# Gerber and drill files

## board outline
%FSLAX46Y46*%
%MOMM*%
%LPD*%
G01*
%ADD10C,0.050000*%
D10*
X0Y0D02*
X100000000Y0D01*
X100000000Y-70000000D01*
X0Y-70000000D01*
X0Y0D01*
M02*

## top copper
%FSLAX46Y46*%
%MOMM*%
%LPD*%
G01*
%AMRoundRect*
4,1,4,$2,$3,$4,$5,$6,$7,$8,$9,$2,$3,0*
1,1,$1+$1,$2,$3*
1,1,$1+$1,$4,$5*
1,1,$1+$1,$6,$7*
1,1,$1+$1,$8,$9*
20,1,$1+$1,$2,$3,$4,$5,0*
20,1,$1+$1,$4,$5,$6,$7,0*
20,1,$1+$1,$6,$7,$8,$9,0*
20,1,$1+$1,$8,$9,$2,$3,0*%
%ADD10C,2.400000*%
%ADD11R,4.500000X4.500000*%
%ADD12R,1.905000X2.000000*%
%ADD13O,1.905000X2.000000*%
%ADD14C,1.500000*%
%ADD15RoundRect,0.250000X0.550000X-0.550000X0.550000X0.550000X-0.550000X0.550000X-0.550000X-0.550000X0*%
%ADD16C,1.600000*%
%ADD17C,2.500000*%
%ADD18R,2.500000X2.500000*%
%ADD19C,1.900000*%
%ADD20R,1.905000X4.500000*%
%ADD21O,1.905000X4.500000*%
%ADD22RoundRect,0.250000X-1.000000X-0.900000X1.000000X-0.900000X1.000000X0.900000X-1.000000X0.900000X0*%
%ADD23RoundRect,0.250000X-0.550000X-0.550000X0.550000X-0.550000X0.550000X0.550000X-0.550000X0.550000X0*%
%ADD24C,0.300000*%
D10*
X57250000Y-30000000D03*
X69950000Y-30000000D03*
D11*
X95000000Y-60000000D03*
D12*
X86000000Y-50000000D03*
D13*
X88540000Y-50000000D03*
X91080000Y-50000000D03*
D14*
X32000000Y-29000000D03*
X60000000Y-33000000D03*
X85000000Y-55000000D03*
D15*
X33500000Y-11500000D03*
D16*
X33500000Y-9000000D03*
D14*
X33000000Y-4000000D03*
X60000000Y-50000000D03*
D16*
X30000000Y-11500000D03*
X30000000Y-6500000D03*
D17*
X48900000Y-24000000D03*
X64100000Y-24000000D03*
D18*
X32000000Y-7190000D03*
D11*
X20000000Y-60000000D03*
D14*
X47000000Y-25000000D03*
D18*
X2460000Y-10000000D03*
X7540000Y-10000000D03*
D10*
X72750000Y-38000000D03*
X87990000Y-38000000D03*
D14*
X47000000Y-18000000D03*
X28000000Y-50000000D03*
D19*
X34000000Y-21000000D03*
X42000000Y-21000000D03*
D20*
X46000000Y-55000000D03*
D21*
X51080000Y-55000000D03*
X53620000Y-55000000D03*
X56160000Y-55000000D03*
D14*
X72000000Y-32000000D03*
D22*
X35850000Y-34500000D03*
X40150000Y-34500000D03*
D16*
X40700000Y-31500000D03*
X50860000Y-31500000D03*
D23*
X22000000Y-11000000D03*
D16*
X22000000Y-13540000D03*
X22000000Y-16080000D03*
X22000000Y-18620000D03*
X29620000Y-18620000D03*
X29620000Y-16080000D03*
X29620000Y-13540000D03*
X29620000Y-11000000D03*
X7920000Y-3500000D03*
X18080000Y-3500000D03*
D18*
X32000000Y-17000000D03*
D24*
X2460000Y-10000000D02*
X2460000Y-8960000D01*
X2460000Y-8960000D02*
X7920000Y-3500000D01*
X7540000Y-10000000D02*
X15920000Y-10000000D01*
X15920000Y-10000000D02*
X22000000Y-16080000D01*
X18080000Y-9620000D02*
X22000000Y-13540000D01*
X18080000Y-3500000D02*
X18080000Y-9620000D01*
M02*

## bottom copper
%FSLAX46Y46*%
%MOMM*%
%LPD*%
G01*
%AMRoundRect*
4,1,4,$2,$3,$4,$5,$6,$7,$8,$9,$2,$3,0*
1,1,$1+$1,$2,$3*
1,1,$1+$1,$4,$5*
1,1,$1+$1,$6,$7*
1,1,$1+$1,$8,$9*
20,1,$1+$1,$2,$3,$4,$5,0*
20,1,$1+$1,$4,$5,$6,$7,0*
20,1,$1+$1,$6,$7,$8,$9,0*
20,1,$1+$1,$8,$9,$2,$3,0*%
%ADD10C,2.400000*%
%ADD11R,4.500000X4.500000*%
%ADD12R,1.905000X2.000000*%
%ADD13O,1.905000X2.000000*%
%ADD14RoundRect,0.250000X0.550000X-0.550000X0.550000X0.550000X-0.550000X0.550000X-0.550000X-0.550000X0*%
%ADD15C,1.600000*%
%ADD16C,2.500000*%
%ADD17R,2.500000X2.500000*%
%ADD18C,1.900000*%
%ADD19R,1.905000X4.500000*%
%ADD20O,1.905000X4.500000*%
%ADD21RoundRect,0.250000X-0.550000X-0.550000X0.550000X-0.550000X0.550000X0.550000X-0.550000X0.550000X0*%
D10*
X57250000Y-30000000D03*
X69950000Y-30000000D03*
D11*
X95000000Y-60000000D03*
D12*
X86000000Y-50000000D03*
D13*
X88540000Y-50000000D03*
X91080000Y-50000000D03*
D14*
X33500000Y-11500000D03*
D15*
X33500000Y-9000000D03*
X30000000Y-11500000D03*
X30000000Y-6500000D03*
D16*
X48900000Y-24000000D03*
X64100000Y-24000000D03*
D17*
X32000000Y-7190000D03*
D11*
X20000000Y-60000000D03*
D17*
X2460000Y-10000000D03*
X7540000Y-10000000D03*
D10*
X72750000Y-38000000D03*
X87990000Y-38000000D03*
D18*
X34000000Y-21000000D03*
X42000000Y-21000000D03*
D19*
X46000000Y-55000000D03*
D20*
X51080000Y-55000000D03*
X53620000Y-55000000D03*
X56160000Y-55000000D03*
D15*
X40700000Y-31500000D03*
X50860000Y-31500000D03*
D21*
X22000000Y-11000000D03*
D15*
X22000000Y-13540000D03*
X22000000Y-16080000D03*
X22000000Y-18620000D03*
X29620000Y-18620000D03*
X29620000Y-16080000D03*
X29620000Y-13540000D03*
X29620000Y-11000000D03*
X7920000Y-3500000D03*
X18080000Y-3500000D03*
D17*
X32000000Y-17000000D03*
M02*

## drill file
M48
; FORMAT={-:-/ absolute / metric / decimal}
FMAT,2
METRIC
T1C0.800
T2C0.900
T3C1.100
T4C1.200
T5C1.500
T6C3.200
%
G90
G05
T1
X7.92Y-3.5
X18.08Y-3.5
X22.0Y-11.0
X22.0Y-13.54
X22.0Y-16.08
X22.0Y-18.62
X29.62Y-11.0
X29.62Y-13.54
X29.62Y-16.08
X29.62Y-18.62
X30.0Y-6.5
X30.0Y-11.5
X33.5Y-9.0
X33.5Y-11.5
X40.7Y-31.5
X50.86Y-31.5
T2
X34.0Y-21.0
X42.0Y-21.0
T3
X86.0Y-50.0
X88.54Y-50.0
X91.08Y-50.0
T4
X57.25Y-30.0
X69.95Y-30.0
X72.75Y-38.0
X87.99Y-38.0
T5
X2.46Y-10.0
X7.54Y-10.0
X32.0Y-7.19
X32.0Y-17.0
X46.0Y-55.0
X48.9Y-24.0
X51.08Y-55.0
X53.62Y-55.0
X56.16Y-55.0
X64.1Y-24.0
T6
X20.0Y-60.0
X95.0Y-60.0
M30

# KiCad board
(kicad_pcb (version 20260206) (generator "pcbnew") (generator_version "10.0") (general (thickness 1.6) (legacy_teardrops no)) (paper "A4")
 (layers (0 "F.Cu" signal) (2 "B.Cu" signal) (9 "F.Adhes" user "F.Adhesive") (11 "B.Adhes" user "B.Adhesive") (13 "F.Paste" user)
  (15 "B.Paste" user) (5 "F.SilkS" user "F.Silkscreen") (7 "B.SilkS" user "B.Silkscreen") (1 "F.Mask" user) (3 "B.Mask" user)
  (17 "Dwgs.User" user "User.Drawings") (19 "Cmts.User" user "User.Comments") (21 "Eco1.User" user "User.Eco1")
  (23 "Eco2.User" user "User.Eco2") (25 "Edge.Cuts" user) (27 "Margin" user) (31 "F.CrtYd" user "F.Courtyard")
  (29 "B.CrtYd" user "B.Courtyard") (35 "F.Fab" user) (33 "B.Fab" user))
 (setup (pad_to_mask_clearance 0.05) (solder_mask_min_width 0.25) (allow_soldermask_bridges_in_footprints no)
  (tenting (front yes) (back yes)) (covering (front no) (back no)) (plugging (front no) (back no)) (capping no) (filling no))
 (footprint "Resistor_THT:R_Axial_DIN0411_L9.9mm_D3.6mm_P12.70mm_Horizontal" (layer "F.Cu") (at 57.25 30)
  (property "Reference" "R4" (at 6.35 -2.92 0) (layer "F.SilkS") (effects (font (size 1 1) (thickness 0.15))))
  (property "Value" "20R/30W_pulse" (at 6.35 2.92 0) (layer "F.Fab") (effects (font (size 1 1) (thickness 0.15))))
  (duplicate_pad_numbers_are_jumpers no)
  (pad "1" thru_hole circle (at 0 0) (size 2.4 2.4) (drill 1.2) (layers "*.Cu" "*.Mask") (remove_unused_layers no) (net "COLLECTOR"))
  (pad "2" thru_hole circle (at 12.7 0) (size 2.4 2.4) (drill 1.2) (layers "*.Cu" "*.Mask") (remove_unused_layers no)
   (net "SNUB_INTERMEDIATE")))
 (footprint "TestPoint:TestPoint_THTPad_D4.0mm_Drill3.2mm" (layer "F.Cu") (at 95 60)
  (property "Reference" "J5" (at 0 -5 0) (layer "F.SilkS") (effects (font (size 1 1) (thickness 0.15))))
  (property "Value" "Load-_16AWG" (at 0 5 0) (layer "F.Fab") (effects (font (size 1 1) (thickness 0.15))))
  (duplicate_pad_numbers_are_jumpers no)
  (pad "1" thru_hole rect (at 0 0) (size 4.5 4.5) (drill 3.2) (layers "*.Cu" "*.Mask") (remove_unused_layers no) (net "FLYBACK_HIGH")))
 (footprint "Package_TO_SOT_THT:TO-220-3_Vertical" (layer "F.Cu") (at 86 50)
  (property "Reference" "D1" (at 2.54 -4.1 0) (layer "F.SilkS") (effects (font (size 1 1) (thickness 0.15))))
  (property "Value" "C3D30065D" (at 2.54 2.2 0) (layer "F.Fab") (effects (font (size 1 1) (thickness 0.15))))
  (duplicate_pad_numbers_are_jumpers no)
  (pad "1" thru_hole rect (at 0 0) (size 1.905 2) (drill 1.1) (layers "*.Cu" "*.Mask") (remove_unused_layers no) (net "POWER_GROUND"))
  (pad "2" thru_hole oval (at 2.54 0) (size 1.905 2) (drill 1.1) (layers "*.Cu" "*.Mask") (remove_unused_layers no) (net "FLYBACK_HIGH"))
  (pad "3" thru_hole oval (at 5.08 0) (size 1.905 2) (drill 1.1) (layers "*.Cu" "*.Mask") (remove_unused_layers no) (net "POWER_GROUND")))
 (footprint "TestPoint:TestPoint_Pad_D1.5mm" (layer "F.Cu") (at 32 29)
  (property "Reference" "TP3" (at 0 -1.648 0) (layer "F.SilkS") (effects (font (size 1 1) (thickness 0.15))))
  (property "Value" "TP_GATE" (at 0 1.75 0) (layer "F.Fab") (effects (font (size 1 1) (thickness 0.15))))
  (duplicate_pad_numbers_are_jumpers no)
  (pad "1" smd circle (at 0 0) (size 1.5 1.5) (layers "F.Cu" "F.Mask") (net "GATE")))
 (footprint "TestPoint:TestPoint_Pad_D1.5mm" (layer "F.Cu") (at 60 33)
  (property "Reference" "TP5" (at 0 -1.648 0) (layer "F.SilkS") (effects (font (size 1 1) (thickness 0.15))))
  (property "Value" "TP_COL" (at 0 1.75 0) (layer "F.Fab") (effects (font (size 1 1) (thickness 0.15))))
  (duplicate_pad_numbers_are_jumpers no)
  (pad "1" smd circle (at 0 0) (size 1.5 1.5) (layers "F.Cu" "F.Mask") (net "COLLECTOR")))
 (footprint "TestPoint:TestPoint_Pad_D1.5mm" (layer "F.Cu") (at 85 55)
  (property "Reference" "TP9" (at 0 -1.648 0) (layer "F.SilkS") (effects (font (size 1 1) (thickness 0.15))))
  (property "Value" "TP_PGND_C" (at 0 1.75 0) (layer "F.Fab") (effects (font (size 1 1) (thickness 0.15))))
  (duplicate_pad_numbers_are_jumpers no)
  (pad "1" smd circle (at 0 0) (size 1.5 1.5) (layers "F.Cu" "F.Mask") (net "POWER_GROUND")))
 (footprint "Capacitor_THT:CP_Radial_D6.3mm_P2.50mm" (layer "F.Cu") (at 33.5 11.5 90)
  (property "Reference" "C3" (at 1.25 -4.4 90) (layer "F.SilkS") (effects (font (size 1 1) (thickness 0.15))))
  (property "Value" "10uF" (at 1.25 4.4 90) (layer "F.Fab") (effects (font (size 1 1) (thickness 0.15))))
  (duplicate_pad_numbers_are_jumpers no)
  (pad "1" thru_hole roundrect (at 0 0 90) (size 1.6 1.6) (drill 0.8) (layers "*.Cu" "*.Mask") (remove_unused_layers no)
   (roundrect_rratio 0.15625) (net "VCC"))
  (pad "2" thru_hole circle (at 2.5 0 90) (size 1.6 1.6) (drill 0.8) (layers "*.Cu" "*.Mask") (remove_unused_layers no)
   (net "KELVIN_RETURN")))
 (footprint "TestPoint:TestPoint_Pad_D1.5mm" (layer "F.Cu") (at 33 4)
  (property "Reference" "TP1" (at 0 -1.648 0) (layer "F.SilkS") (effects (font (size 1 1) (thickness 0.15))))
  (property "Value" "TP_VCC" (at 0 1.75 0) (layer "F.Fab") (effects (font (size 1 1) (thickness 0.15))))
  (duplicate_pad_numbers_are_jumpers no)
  (pad "1" smd circle (at 0 0) (size 1.5 1.5) (layers "F.Cu" "F.Mask") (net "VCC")))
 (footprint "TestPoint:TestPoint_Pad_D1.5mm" (layer "F.Cu") (at 60 50)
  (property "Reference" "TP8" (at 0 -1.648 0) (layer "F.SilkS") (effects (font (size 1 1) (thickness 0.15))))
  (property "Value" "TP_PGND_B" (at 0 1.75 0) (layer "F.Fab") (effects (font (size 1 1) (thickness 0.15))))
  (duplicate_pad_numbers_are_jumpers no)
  (pad "1" smd circle (at 0 0) (size 1.5 1.5) (layers "F.Cu" "F.Mask") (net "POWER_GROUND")))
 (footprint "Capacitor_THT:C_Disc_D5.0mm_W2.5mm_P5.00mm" (layer "F.Cu") (at 30 11.5 90)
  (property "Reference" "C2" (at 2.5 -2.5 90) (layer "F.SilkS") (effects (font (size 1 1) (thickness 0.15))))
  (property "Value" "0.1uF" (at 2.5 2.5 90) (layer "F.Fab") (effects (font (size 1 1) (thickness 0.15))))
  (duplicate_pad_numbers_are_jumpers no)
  (pad "1" thru_hole circle (at 0 0 90) (size 1.6 1.6) (drill 0.8) (layers "*.Cu" "*.Mask") (remove_unused_layers no) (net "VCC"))
  (pad "2" thru_hole circle (at 5 0 90) (size 1.6 1.6) (drill 0.8) (layers "*.Cu" "*.Mask") (remove_unused_layers no) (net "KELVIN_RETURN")))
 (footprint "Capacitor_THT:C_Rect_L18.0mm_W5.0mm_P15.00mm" (layer "F.Cu") (at 56.5 24)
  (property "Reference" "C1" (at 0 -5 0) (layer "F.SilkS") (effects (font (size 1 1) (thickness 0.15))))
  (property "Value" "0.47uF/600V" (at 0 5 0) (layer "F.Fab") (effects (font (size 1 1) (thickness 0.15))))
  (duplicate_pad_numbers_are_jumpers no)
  (pad "1" thru_hole circle (at -7.6 0) (size 2.5 2.5) (drill 1.5) (layers "*.Cu" "*.Mask") (remove_unused_layers no) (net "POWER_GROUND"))
  (pad "2" thru_hole circle (at 7.6 0) (size 2.5 2.5) (drill 1.5) (layers "*.Cu" "*.Mask") (remove_unused_layers no)
   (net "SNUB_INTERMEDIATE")))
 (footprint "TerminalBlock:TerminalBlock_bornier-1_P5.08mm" (layer "F.Cu") (at 32 7.19)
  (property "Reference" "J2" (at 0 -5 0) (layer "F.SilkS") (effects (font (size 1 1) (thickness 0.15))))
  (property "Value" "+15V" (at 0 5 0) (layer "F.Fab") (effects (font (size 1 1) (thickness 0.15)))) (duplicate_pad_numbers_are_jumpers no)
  (pad "1" thru_hole rect (at 0 0) (size 2.5 2.5) (drill 1.5) (layers "*.Cu" "*.Mask") (remove_unused_layers no) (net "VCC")))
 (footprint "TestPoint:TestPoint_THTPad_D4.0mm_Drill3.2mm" (layer "F.Cu") (at 20 60)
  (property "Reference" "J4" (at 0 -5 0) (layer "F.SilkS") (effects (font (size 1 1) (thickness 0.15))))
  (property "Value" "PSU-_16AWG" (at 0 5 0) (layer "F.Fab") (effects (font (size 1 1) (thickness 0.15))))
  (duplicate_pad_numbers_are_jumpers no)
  (pad "1" thru_hole rect (at 0 0) (size 4.5 4.5) (drill 3.2) (layers "*.Cu" "*.Mask") (remove_unused_layers no) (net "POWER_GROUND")))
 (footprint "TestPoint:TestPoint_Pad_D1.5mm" (layer "F.Cu") (at 47 25)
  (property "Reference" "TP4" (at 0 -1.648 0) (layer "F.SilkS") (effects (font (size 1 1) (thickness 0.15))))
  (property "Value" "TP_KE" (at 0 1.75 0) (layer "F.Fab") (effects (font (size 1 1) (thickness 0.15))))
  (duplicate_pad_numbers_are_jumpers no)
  (pad "1" smd circle (at 0 0) (size 1.5 1.5) (layers "F.Cu" "F.Mask") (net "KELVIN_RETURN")))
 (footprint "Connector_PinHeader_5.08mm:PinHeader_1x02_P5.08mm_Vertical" (layer "F.Cu") (at 5 10 90)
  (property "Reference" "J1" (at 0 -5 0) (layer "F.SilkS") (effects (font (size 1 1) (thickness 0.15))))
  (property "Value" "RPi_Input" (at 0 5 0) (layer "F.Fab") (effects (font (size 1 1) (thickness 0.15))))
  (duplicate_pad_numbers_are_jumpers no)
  (pad "1" thru_hole rect (at 0 -2.54) (size 2.5 2.5) (drill 1.5) (layers "*.Cu" "*.Mask") (remove_unused_layers no) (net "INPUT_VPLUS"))
  (pad "2" thru_hole rect (at 0 2.54) (size 2.5 2.5) (drill 1.5) (layers "*.Cu" "*.Mask") (remove_unused_layers no) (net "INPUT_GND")))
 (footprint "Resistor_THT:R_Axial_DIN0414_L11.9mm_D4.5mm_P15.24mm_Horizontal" (layer "F.Cu") (at 72.75 38)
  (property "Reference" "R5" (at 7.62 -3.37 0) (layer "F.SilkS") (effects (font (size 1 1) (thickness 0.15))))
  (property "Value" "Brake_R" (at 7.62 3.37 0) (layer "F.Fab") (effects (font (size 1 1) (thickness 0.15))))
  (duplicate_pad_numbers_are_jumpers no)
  (pad "1" thru_hole circle (at 0 0) (size 2.4 2.4) (drill 1.2) (layers "*.Cu" "*.Mask") (remove_unused_layers no) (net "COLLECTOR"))
  (pad "2" thru_hole circle (at 15.24 0) (size 2.4 2.4) (drill 1.2) (layers "*.Cu" "*.Mask") (remove_unused_layers no) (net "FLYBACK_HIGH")))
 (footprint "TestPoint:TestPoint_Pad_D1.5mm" (layer "F.Cu") (at 47 18)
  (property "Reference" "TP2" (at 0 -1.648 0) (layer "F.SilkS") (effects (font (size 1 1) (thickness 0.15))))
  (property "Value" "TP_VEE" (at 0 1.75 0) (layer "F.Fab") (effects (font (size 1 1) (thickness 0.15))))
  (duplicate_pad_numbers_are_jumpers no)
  (pad "1" smd circle (at 0 0) (size 1.5 1.5) (layers "F.Cu" "F.Mask") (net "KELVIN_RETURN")))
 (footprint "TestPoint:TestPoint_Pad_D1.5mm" (layer "F.Cu") (at 28 50)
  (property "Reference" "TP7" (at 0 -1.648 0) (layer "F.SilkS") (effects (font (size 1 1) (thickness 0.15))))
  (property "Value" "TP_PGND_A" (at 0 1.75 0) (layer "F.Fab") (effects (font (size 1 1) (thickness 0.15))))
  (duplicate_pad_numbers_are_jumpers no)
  (pad "1" smd circle (at 0 0) (size 1.5 1.5) (layers "F.Cu" "F.Mask") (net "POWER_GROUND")))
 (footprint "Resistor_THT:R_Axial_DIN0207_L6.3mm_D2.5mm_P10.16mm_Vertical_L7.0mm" (layer "F.Cu") (at 38 21 90)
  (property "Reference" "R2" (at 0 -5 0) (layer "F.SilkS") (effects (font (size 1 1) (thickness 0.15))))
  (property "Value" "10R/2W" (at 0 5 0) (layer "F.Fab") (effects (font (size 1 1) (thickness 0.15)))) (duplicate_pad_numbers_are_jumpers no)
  (pad "1" thru_hole circle (at 0 -4) (size 1.9 1.9) (drill 0.9) (layers "*.Cu" "*.Mask") (remove_unused_layers no) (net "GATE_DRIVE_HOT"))
  (pad "2" thru_hole circle (at 0 4) (size 1.9 1.9) (drill 0.9) (layers "*.Cu" "*.Mask") (remove_unused_layers no) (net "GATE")))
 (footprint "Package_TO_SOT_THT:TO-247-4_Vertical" (layer "F.Cu") (at 46 55)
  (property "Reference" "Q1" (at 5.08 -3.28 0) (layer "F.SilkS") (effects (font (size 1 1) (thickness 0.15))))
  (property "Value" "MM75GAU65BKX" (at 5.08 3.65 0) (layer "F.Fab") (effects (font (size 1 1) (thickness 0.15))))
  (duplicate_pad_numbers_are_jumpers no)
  (pad "1" thru_hole rect (at 0 0) (size 1.905 4.5) (drill 1.5) (layers "*.Cu" "*.Mask") (remove_unused_layers no) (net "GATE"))
  (pad "2" thru_hole oval (at 5.08 0) (size 1.905 4.5) (drill 1.5) (layers "*.Cu" "*.Mask") (remove_unused_layers no) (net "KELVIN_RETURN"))
  (pad "3" thru_hole oval (at 7.62 0) (size 1.905 4.5) (drill 1.5) (layers "*.Cu" "*.Mask") (remove_unused_layers no) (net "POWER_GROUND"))
  (pad "4" thru_hole oval (at 10.16 0) (size 1.905 4.5) (drill 1.5) (layers "*.Cu" "*.Mask") (remove_unused_layers no) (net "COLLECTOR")))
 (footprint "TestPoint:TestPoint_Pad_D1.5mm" (layer "F.Cu") (at 72 32)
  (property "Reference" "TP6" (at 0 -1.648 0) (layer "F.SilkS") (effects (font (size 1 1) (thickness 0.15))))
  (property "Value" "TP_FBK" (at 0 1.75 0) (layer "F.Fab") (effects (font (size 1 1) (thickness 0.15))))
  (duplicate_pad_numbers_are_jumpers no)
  (pad "1" smd circle (at 0 0) (size 1.5 1.5) (layers "F.Cu" "F.Mask") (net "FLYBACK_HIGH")))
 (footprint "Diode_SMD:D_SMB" (layer "F.Cu") (at 38 34.5)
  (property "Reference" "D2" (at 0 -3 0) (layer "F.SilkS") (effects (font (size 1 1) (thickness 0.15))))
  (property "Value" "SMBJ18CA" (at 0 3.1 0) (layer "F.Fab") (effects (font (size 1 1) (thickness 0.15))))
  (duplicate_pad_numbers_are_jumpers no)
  (pad "1" smd roundrect (at -2.15 0) (size 2.5 2.3) (layers "F.Cu" "F.Mask" "F.Paste") (roundrect_rratio 0.1086956522) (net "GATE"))
  (pad "2" smd roundrect (at 2.15 0) (size 2.5 2.3) (layers "F.Cu" "F.Mask" "F.Paste") (roundrect_rratio 0.1086956522) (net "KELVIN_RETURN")))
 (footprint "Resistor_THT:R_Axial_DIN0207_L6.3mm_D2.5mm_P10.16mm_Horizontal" (layer "F.Cu") (at 40.7 31.5)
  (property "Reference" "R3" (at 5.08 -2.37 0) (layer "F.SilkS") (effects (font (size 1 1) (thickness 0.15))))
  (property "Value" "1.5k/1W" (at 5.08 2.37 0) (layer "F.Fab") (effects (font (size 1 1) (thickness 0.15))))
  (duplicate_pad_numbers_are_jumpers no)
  (pad "1" thru_hole circle (at 0 0) (size 1.6 1.6) (drill 0.8) (layers "*.Cu" "*.Mask") (remove_unused_layers no) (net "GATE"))
  (pad "2" thru_hole circle (at 10.16 0) (size 1.6 1.6) (drill 0.8) (layers "*.Cu" "*.Mask") (remove_unused_layers no) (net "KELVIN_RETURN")))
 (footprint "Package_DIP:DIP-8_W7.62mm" (layer "F.Cu") (at 22 11)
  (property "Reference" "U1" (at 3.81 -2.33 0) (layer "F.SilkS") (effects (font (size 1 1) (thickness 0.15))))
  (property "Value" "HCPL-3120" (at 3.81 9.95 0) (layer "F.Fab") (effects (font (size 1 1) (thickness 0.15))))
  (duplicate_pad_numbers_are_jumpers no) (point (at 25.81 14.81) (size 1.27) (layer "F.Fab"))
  (pad "1" thru_hole roundrect (at 0 0) (size 1.6 1.6) (drill 0.8) (layers "*.Cu" "*.Mask") (remove_unused_layers no)
   (roundrect_rratio 0.15625))
  (pad "2" thru_hole circle (at 0 2.54) (size 1.6 1.6) (drill 0.8) (layers "*.Cu" "*.Mask") (remove_unused_layers no) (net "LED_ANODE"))
  (pad "3" thru_hole circle (at 0 5.08) (size 1.6 1.6) (drill 0.8) (layers "*.Cu" "*.Mask") (remove_unused_layers no) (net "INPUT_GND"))
  (pad "4" thru_hole circle (at 0 7.62) (size 1.6 1.6) (drill 0.8) (layers "*.Cu" "*.Mask") (remove_unused_layers no))
  (pad "5" thru_hole circle (at 7.62 7.62) (size 1.6 1.6) (drill 0.8) (layers "*.Cu" "*.Mask") (remove_unused_layers no)
   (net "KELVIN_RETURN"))
  (pad "6" thru_hole circle (at 7.62 5.08) (size 1.6 1.6) (drill 0.8) (layers "*.Cu" "*.Mask") (remove_unused_layers no)
   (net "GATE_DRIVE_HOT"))
  (pad "7" thru_hole circle (at 7.62 2.54) (size 1.6 1.6) (drill 0.8) (layers "*.Cu" "*.Mask") (remove_unused_layers no)
   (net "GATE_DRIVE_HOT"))
  (pad "8" thru_hole circle (at 7.62 0) (size 1.6 1.6) (drill 0.8) (layers "*.Cu" "*.Mask") (remove_unused_layers no) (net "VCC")))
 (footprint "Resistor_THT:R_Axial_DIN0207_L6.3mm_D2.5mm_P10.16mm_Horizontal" (layer "F.Cu") (at 7.92 3.5)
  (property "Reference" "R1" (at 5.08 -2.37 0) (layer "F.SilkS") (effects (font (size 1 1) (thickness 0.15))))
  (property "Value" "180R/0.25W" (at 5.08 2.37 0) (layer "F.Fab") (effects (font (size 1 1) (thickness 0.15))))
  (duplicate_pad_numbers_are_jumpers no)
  (pad "1" thru_hole circle (at 0 0) (size 1.6 1.6) (drill 0.8) (layers "*.Cu" "*.Mask") (remove_unused_layers no) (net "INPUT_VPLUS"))
  (pad "2" thru_hole circle (at 10.16 0) (size 1.6 1.6) (drill 0.8) (layers "*.Cu" "*.Mask") (remove_unused_layers no) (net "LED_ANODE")))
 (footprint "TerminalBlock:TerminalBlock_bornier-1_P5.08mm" (layer "F.Cu") (at 32 17)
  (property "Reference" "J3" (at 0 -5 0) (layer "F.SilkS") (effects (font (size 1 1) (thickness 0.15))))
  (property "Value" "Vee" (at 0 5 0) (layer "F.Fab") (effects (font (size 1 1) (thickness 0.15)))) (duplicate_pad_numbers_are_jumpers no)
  (pad "1" thru_hole rect (at 0 0) (size 2.5 2.5) (drill 1.5) (layers "*.Cu" "*.Mask") (remove_unused_layers no) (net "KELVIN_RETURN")))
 (gr_rect (start 0 0) (end 100 70) (stroke (width 0.05) (type solid)) (fill no) (layer "Edge.Cuts"))
 (segment (start 2.46 10) (end 2.46 8.96) (width 0.3) (layer "F.Cu") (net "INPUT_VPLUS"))
 (segment (start 2.46 8.96) (end 7.92 3.5) (width 0.3) (layer "F.Cu") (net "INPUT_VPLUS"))
 (segment (start 7.54 10) (end 15.92 10) (width 0.3) (layer "F.Cu") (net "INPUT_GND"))
 (segment (start 15.92 10) (end 22 16.08) (width 0.3) (layer "F.Cu") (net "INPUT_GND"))
 (segment (start 18.08 9.62) (end 22 13.54) (width 0.3) (layer "F.Cu") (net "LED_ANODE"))
 (segment (start 18.08 3.5) (end 18.08 9.62) (width 0.3) (layer "F.Cu") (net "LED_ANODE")))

